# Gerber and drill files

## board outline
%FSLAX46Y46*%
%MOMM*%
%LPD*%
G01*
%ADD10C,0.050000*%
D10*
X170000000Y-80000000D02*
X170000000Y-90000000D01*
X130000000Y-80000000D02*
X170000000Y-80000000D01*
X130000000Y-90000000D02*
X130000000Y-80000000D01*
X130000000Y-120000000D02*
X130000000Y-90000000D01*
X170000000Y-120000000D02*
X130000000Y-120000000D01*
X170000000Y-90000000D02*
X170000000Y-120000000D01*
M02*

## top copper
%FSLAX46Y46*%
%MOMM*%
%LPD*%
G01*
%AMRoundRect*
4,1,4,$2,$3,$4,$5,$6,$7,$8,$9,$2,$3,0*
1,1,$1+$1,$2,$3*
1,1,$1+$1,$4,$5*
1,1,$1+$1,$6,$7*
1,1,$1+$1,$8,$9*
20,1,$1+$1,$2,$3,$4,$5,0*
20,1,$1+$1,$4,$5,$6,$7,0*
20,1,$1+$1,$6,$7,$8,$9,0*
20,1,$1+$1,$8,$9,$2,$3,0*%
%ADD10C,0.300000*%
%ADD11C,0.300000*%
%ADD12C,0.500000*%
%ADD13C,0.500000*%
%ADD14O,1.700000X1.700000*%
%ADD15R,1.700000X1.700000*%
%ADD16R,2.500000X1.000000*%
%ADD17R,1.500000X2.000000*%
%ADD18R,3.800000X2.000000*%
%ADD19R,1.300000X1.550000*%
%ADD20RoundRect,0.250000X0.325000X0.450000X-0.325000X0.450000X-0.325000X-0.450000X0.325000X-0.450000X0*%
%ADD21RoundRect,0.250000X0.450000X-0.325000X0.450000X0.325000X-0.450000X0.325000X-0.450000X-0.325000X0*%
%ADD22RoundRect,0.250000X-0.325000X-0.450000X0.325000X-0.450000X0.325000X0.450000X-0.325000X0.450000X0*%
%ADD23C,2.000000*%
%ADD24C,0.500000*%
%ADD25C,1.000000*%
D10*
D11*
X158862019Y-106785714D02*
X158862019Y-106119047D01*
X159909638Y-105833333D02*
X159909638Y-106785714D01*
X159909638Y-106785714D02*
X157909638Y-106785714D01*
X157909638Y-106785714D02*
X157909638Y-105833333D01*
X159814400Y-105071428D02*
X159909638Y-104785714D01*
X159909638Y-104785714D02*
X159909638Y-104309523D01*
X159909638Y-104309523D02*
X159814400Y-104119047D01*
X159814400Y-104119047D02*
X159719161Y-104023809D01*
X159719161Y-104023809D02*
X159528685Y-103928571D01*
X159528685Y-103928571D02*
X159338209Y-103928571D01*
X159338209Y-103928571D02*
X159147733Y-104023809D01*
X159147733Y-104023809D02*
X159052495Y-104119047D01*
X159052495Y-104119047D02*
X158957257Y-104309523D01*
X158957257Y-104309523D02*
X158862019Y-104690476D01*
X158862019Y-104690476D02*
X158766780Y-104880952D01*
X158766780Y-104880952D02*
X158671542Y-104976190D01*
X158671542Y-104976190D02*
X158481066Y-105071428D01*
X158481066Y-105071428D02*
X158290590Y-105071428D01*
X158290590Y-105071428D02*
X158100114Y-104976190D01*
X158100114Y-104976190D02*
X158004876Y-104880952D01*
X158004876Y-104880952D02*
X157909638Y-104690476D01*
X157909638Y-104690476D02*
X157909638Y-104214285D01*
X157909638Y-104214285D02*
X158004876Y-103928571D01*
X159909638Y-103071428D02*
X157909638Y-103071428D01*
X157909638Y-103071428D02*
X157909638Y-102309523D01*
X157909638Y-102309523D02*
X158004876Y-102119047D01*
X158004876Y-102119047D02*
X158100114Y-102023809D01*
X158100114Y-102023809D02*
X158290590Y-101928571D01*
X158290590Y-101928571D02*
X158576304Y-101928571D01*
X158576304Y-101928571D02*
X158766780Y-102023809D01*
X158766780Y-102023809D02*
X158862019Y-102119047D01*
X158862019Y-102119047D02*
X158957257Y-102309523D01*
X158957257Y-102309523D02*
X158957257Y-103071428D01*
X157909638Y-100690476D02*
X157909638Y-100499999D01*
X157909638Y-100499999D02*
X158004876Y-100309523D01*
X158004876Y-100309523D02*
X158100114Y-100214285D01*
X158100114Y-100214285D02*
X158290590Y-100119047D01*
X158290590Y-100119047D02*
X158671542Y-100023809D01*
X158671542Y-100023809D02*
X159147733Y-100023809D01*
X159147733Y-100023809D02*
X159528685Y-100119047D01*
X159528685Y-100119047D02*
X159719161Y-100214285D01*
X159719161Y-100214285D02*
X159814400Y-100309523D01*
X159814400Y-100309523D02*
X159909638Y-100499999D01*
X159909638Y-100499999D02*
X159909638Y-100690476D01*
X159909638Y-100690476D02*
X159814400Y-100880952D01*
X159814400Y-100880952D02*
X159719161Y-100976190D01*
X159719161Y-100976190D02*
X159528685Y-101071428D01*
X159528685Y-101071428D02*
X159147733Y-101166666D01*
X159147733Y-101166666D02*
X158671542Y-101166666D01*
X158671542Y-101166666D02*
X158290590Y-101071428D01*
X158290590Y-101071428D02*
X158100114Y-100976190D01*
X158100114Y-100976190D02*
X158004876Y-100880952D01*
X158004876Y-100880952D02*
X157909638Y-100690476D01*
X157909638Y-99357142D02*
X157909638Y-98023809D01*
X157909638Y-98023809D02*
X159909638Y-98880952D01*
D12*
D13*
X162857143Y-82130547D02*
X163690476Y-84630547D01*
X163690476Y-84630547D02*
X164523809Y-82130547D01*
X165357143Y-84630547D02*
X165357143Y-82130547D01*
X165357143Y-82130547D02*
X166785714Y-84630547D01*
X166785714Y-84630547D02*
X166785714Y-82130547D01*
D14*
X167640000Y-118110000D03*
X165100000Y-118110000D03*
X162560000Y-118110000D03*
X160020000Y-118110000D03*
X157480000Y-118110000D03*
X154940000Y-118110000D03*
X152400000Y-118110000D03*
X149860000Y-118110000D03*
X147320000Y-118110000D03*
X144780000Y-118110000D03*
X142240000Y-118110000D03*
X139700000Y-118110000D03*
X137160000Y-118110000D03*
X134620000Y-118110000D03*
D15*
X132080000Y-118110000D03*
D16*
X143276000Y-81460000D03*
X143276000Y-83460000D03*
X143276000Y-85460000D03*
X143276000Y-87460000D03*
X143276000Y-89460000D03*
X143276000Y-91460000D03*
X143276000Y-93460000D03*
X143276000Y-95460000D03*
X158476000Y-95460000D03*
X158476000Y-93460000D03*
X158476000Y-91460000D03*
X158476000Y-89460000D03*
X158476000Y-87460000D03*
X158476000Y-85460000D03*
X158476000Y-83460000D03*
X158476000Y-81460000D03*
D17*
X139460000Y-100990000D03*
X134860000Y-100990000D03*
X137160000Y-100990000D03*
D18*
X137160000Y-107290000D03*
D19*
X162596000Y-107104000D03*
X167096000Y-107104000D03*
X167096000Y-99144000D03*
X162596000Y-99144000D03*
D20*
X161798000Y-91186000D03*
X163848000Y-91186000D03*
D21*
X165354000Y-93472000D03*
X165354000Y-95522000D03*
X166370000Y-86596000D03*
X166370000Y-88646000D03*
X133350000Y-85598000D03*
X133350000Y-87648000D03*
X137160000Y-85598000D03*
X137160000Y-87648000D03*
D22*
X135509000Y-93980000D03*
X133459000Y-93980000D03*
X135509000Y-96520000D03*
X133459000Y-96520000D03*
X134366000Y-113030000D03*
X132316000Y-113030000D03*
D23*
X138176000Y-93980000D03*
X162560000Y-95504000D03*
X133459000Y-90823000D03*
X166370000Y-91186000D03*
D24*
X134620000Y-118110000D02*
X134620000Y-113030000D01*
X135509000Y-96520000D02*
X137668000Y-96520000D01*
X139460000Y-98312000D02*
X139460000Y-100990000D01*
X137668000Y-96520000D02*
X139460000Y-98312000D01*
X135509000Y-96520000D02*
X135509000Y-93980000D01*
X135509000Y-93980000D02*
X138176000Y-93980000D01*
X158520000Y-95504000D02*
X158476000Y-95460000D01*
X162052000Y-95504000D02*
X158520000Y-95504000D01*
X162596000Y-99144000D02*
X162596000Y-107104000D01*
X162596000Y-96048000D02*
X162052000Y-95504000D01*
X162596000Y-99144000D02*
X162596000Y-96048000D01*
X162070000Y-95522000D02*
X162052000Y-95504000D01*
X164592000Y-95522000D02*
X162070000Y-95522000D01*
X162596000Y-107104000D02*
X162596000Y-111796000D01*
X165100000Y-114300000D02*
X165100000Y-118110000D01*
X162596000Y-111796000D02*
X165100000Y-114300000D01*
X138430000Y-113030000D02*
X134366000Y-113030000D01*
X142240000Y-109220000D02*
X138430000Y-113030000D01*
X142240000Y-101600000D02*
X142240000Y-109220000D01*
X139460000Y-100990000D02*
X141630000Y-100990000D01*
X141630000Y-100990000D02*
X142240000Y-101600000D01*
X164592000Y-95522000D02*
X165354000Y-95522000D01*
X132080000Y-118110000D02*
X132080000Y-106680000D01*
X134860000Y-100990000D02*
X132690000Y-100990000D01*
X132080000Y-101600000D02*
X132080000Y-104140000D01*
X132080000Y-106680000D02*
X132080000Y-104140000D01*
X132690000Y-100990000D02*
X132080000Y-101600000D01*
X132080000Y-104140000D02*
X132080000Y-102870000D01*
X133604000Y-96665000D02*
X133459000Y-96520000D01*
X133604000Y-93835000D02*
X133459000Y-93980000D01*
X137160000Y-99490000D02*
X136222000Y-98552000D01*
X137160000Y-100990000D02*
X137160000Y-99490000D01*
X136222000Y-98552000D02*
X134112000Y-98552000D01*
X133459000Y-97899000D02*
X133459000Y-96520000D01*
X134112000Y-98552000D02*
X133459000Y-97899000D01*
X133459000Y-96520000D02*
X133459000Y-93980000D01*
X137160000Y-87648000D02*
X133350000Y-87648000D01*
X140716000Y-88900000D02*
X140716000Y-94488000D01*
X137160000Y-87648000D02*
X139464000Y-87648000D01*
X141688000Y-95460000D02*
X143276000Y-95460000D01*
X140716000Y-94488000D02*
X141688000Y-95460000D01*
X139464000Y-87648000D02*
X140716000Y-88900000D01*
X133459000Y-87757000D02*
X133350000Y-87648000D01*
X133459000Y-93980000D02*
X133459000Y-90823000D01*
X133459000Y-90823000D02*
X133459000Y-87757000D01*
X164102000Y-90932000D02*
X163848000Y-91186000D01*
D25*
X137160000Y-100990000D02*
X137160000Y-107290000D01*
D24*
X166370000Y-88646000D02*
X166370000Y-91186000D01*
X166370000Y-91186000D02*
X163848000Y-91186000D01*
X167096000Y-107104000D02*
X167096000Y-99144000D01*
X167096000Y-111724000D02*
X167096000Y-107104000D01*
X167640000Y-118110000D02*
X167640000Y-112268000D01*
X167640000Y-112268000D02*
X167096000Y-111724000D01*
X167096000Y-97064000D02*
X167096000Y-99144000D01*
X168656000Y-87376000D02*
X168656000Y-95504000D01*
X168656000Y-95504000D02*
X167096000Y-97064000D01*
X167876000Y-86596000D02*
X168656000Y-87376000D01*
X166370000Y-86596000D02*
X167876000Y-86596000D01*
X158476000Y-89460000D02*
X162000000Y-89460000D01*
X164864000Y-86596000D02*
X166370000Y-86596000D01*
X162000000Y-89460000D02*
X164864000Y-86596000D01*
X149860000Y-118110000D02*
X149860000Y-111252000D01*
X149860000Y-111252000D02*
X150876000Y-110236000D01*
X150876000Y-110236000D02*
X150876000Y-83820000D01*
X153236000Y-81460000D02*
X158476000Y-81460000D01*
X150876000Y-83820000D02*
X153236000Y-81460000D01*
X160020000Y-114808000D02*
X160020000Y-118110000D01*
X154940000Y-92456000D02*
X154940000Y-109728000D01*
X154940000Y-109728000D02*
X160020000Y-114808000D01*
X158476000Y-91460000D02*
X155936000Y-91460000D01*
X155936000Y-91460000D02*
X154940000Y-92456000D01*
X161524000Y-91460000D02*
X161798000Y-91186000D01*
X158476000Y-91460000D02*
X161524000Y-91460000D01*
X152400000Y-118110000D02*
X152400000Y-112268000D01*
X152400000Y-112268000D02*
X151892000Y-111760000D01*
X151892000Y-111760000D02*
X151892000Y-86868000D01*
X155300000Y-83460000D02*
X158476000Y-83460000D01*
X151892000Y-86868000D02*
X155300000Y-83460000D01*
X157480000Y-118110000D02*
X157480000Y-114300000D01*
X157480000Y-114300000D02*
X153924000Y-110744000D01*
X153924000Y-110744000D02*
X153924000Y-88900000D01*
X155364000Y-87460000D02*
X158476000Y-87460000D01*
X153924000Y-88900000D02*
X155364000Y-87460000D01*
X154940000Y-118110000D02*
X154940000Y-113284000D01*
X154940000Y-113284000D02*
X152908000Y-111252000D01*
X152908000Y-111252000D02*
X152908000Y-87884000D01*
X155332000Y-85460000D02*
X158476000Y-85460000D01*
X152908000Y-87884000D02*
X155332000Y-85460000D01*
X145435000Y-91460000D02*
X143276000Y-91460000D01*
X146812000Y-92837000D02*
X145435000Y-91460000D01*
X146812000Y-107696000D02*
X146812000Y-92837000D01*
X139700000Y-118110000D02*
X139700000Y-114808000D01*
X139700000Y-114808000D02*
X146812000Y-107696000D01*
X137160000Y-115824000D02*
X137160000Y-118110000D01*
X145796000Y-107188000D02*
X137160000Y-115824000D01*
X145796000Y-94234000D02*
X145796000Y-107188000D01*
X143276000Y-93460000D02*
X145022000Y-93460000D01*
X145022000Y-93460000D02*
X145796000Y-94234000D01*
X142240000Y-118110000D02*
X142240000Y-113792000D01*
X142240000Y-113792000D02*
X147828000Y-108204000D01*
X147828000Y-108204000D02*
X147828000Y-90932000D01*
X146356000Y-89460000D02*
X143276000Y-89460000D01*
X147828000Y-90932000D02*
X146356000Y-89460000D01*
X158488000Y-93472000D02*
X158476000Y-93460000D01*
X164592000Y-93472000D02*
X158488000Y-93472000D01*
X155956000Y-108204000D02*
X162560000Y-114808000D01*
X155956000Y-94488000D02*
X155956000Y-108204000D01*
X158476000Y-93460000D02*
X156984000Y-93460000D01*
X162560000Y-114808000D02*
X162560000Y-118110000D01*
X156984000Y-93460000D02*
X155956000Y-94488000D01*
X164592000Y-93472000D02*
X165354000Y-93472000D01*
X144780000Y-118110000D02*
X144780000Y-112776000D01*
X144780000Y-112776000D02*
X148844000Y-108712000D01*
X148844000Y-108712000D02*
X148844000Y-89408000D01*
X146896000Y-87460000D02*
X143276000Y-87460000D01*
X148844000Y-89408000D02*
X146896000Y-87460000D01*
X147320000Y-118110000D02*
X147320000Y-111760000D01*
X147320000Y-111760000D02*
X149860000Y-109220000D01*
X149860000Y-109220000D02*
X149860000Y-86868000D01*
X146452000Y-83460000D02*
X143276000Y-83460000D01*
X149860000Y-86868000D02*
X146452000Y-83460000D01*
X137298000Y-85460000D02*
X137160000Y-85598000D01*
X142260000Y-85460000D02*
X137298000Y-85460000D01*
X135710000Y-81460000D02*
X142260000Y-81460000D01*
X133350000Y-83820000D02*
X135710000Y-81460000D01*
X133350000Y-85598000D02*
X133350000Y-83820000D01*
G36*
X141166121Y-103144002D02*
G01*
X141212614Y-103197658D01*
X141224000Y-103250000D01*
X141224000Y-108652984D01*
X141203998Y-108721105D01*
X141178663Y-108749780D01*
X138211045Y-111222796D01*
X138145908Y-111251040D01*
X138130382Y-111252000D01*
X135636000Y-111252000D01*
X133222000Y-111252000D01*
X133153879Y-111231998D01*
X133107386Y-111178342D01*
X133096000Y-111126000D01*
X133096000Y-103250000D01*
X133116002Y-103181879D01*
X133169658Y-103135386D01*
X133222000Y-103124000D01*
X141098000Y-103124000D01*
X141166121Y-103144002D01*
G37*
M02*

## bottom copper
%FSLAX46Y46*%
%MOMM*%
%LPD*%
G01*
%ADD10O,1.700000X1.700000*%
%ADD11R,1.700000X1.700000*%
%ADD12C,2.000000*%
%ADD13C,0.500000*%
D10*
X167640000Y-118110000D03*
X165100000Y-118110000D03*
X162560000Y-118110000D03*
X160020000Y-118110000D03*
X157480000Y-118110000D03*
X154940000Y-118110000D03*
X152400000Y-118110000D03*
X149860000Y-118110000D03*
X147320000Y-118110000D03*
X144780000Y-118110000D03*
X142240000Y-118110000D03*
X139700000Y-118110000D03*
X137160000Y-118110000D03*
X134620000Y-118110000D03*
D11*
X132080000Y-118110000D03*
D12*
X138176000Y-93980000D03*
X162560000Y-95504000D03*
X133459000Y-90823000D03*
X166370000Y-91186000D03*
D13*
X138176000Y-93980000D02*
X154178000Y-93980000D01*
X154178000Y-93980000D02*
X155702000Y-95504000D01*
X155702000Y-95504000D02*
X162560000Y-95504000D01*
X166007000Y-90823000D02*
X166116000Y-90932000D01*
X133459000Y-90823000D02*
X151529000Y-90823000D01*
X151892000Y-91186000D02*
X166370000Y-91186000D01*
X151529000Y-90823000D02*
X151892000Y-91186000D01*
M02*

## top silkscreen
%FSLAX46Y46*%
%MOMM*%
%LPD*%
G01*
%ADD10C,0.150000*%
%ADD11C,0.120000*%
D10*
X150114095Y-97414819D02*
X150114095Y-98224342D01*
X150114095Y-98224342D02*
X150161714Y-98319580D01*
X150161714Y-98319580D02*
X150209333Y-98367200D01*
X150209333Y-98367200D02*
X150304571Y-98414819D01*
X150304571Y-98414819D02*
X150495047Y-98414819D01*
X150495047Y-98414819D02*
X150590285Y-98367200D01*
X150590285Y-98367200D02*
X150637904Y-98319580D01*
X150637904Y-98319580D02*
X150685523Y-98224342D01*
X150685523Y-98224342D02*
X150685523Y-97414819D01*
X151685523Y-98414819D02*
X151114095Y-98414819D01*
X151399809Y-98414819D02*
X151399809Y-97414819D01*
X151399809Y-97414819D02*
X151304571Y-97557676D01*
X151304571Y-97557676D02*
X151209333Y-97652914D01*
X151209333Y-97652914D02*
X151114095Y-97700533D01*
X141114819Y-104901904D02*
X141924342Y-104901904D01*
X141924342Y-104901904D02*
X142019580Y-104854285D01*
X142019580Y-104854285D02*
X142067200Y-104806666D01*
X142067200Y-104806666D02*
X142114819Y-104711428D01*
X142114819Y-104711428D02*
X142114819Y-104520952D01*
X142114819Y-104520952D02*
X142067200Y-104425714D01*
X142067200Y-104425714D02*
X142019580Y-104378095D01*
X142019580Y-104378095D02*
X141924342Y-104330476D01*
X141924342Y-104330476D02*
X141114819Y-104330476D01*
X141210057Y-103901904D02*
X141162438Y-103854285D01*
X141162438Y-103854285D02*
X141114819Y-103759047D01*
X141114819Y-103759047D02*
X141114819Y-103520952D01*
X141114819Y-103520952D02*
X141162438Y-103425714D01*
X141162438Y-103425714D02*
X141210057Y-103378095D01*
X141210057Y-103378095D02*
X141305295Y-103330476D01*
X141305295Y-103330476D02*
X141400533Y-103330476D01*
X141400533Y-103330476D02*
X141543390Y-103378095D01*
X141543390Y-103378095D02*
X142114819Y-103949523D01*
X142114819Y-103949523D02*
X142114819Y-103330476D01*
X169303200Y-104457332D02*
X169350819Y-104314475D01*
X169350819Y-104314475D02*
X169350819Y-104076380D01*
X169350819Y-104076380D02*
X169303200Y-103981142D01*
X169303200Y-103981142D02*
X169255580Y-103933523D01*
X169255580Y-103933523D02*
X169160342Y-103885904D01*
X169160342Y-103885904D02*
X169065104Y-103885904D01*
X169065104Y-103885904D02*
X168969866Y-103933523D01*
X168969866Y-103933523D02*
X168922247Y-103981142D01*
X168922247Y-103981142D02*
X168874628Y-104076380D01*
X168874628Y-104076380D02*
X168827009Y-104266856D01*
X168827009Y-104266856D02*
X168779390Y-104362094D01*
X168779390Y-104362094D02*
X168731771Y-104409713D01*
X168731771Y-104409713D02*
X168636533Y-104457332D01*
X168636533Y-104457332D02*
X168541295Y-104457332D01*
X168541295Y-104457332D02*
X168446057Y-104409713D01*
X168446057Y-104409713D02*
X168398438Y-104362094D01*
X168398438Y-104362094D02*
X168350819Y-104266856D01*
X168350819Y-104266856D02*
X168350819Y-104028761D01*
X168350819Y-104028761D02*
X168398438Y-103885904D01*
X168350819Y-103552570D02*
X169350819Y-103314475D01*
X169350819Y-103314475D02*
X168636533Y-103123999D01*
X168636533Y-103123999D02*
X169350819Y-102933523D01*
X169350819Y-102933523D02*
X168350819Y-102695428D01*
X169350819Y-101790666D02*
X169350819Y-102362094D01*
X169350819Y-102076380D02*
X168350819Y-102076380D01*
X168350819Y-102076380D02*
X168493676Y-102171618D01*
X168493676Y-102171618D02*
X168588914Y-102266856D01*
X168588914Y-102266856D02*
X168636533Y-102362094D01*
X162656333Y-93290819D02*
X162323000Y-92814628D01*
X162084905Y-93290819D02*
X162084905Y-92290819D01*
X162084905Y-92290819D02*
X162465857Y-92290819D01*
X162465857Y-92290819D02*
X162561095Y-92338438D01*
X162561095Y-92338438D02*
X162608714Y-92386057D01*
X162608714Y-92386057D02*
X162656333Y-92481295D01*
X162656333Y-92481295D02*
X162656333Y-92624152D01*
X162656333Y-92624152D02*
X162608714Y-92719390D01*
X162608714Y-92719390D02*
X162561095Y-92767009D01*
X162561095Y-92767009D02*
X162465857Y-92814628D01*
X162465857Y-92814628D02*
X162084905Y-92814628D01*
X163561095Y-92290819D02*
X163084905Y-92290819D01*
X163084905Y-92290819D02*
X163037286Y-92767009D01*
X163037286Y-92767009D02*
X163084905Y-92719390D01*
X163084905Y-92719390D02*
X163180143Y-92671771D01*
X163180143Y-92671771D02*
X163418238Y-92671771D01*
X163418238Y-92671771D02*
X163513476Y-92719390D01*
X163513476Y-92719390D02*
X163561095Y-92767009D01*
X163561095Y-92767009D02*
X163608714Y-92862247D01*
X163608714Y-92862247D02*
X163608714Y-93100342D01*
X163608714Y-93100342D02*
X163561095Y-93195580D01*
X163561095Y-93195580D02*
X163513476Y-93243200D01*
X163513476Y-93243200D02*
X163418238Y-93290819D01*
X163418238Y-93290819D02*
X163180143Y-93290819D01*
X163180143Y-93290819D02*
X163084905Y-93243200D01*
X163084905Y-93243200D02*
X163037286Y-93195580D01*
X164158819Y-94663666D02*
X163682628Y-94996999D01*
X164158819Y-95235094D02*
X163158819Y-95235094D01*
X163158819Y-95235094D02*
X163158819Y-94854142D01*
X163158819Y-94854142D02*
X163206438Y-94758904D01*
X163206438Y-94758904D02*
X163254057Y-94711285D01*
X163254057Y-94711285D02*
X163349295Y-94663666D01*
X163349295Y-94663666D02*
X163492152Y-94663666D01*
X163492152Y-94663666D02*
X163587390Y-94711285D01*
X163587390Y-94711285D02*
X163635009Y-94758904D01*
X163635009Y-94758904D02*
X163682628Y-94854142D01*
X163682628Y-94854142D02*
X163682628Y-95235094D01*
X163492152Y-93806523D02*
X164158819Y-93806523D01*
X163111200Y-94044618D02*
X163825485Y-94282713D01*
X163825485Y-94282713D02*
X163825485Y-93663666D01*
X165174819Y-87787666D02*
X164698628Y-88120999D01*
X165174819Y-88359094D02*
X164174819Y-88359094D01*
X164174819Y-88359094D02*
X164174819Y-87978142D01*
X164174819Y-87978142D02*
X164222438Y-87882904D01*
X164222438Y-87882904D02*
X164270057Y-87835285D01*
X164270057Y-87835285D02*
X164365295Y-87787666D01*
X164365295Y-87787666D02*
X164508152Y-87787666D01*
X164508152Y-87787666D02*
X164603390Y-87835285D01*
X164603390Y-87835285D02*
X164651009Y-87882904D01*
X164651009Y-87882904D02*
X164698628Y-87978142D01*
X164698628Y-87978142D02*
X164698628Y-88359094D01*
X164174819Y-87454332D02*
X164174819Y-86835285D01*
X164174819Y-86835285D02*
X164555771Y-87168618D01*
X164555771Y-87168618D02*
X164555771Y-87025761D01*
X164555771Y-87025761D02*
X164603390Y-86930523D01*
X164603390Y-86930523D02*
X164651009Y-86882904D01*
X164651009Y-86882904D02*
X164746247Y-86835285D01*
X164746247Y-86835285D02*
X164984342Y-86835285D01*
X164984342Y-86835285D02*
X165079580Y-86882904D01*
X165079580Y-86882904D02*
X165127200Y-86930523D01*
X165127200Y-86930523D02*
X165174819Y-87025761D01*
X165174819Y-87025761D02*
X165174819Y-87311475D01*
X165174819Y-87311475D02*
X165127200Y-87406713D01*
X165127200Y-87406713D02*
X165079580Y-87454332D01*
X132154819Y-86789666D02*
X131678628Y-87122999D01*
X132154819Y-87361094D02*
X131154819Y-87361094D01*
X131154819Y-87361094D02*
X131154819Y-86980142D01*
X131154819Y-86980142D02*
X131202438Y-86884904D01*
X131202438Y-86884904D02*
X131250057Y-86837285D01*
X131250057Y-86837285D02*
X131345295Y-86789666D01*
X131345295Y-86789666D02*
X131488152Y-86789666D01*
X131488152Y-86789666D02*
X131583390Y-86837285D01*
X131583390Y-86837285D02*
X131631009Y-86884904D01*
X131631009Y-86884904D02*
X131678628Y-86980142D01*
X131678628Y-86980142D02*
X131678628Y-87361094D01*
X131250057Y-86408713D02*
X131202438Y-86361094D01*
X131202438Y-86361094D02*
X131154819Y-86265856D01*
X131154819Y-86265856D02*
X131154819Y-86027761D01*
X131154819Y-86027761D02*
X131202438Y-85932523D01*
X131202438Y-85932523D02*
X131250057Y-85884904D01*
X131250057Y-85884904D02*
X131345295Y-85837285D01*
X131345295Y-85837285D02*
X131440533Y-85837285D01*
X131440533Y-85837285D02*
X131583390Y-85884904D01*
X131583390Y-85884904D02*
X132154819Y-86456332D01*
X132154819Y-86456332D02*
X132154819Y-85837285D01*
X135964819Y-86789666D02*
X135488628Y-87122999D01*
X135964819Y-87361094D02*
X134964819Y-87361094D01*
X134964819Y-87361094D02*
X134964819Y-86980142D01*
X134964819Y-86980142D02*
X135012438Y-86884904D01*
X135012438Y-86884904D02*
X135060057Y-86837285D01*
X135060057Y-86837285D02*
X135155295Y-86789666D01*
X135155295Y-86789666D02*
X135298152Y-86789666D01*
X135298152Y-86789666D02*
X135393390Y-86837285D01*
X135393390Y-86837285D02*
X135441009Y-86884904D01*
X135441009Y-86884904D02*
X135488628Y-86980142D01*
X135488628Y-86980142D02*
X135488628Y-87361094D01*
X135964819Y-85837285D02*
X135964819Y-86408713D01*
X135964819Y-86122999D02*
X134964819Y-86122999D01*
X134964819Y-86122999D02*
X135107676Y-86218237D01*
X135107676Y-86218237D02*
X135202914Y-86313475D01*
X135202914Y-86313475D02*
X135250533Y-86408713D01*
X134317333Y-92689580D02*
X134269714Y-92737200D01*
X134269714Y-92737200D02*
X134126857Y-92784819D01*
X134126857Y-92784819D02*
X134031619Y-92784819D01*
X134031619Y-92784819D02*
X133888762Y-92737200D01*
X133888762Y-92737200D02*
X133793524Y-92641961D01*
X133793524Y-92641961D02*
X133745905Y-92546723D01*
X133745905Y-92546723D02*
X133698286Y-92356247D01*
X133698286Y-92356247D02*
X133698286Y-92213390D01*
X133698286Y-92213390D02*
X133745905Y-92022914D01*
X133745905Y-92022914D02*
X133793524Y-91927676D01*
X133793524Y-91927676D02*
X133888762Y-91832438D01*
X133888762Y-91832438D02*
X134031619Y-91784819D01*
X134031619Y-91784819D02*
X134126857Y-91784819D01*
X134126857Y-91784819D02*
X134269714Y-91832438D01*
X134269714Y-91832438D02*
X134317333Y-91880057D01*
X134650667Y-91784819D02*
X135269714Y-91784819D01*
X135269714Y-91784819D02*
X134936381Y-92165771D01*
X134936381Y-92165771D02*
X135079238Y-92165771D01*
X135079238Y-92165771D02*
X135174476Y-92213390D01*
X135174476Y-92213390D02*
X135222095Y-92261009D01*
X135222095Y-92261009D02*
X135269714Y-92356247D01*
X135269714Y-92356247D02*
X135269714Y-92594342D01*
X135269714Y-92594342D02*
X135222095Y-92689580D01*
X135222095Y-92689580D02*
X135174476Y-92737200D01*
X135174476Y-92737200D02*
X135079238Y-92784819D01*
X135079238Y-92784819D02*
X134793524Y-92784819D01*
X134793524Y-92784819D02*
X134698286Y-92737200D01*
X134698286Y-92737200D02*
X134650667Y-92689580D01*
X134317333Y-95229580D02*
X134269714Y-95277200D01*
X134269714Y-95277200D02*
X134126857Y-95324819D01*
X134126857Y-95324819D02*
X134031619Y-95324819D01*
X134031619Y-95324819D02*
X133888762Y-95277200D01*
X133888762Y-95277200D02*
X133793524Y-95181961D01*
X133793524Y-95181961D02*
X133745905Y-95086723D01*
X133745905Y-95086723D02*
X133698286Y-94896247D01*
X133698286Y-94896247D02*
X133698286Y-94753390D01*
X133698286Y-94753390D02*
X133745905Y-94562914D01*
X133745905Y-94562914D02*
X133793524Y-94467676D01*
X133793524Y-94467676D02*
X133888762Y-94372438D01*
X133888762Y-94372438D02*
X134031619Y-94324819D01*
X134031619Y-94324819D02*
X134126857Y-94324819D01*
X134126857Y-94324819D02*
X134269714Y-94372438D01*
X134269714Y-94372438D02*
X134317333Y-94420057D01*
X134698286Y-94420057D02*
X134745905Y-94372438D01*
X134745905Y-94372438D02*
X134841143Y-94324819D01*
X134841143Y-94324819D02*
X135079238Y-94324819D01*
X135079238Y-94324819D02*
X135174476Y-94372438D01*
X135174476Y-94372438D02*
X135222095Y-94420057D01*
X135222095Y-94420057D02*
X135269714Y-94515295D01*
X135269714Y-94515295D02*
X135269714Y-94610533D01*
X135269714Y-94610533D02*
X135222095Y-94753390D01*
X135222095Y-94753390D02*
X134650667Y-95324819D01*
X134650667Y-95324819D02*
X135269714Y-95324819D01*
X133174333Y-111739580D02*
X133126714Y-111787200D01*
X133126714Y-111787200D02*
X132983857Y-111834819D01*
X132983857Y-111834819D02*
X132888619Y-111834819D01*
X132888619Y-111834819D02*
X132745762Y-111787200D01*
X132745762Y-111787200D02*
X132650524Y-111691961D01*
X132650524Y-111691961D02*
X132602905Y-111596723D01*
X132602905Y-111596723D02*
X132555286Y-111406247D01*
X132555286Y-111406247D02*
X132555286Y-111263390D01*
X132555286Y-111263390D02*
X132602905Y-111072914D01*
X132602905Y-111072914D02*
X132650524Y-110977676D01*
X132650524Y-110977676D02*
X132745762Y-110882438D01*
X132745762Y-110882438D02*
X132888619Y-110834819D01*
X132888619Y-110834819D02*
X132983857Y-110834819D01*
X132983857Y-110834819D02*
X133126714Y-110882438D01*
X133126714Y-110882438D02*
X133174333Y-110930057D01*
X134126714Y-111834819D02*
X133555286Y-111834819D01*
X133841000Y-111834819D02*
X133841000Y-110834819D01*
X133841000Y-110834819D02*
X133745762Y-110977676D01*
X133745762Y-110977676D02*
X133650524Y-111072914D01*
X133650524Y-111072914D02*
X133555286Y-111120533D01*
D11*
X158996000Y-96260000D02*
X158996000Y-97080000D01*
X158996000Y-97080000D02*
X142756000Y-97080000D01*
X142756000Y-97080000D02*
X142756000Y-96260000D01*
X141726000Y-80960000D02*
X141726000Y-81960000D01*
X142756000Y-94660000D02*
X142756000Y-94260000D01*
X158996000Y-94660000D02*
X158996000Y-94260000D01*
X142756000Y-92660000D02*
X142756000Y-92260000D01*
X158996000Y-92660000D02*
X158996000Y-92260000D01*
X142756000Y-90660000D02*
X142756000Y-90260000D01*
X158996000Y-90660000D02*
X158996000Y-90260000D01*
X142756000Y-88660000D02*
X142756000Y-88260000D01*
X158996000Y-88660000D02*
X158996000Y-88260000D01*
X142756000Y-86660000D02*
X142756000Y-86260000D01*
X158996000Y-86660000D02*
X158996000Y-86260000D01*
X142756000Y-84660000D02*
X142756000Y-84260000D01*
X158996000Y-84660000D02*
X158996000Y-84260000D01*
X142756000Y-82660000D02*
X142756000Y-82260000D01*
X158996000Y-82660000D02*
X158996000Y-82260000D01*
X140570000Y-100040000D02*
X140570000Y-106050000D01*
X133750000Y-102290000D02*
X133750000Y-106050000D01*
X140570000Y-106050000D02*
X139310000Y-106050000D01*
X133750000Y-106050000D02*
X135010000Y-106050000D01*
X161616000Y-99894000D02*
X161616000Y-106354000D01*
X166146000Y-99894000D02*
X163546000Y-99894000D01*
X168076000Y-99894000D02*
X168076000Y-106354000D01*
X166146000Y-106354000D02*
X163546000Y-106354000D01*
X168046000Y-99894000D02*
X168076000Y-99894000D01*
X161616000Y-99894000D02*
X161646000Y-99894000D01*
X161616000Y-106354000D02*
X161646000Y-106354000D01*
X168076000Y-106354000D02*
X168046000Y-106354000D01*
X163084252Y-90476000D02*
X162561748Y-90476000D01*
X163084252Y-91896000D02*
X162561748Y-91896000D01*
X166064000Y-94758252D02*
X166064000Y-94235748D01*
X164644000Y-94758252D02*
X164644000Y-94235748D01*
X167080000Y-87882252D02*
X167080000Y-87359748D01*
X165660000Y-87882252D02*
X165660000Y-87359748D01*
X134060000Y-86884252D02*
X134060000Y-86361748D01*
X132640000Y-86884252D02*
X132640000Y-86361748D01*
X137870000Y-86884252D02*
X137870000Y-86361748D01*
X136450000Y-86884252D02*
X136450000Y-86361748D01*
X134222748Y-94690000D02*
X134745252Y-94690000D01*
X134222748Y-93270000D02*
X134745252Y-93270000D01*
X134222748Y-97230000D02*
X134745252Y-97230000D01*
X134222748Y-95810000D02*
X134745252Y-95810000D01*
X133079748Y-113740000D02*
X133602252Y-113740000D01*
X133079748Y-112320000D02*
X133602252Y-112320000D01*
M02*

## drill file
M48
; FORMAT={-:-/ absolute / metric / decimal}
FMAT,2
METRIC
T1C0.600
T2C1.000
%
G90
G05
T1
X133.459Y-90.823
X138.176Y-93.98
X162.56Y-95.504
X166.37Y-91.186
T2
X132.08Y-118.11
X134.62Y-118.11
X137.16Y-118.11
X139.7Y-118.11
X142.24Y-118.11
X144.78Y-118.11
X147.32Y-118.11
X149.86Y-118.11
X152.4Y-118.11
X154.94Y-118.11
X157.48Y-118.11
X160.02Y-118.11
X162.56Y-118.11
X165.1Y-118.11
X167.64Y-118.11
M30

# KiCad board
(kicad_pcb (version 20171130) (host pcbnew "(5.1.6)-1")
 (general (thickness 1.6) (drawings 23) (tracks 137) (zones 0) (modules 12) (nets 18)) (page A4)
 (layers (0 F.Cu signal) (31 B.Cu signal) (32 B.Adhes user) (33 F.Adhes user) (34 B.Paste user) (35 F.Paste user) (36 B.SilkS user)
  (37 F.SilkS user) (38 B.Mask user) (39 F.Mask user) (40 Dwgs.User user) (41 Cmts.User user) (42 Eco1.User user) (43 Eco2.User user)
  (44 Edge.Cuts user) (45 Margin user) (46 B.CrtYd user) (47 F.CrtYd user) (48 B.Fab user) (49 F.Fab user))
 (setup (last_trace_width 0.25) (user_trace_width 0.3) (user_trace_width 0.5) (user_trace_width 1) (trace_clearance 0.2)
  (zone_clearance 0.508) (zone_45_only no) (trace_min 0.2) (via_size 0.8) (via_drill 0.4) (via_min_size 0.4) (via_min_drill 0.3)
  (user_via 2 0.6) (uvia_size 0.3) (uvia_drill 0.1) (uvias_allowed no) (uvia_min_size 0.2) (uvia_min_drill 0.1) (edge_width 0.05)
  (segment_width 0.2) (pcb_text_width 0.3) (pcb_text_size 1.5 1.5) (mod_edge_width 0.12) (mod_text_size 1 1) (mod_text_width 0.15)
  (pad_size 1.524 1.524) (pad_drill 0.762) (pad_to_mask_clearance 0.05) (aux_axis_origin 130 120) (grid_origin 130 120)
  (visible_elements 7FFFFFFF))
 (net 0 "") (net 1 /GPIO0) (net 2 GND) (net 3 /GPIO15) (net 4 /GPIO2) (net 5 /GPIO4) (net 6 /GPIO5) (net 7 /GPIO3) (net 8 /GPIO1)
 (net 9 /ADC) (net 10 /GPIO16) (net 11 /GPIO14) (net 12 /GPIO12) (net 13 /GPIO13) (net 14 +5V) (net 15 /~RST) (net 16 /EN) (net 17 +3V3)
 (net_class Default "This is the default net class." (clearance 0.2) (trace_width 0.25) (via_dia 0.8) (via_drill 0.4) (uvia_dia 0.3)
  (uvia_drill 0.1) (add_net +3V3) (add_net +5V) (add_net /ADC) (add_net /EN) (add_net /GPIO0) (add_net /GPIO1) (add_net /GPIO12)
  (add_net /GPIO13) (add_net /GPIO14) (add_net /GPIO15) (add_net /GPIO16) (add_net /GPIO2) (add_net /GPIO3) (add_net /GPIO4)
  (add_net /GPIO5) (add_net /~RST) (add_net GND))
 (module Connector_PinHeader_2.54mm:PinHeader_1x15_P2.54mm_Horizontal (layer B.Cu) (at 132.08 118.11 270)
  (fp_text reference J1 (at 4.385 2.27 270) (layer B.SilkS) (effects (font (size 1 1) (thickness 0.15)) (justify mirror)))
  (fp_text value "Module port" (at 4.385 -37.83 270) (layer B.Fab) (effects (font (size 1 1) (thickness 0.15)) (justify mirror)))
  (pad 15 thru_hole oval (at 0 -35.56 270) (size 1.7 1.7) (drill 1) (layers *.Cu *.Mask) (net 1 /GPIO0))
  (pad 14 thru_hole oval (at 0 -33.02 270) (size 1.7 1.7) (drill 1) (layers *.Cu *.Mask) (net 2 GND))
  (pad 13 thru_hole oval (at 0 -30.48 270) (size 1.7 1.7) (drill 1) (layers *.Cu *.Mask) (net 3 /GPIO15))
  (pad 12 thru_hole oval (at 0 -27.94 270) (size 1.7 1.7) (drill 1) (layers *.Cu *.Mask) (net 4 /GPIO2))
  (pad 11 thru_hole oval (at 0 -25.4 270) (size 1.7 1.7) (drill 1) (layers *.Cu *.Mask) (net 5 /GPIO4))
  (pad 10 thru_hole oval (at 0 -22.86 270) (size 1.7 1.7) (drill 1) (layers *.Cu *.Mask) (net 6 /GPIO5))
  (pad 9 thru_hole oval (at 0 -20.32 270) (size 1.7 1.7) (drill 1) (layers *.Cu *.Mask) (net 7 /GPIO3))
  (pad 8 thru_hole oval (at 0 -17.78 270) (size 1.7 1.7) (drill 1) (layers *.Cu *.Mask) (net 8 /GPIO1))
  (pad 7 thru_hole oval (at 0 -15.24 270) (size 1.7 1.7) (drill 1) (layers *.Cu *.Mask) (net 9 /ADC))
  (pad 6 thru_hole oval (at 0 -12.7 270) (size 1.7 1.7) (drill 1) (layers *.Cu *.Mask) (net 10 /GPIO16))
  (pad 5 thru_hole oval (at 0 -10.16 270) (size 1.7 1.7) (drill 1) (layers *.Cu *.Mask) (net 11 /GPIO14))
  (pad 4 thru_hole oval (at 0 -7.62 270) (size 1.7 1.7) (drill 1) (layers *.Cu *.Mask) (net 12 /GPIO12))
  (pad 3 thru_hole oval (at 0 -5.08 270) (size 1.7 1.7) (drill 1) (layers *.Cu *.Mask) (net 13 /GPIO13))
  (pad 2 thru_hole oval (at 0 -2.54 270) (size 1.7 1.7) (drill 1) (layers *.Cu *.Mask) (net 2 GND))
  (pad 1 thru_hole rect (at 0 0 270) (size 1.7 1.7) (drill 1) (layers *.Cu *.Mask) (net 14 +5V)))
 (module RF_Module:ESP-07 (layer F.Cu) (at 150.876 86.36)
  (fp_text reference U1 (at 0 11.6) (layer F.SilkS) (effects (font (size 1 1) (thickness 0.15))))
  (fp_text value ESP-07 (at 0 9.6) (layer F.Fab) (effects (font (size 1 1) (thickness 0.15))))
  (fp_line (start 8.12 9.9) (end 8.12 10.72) (layer F.SilkS) (width 0.12))
  (fp_line (start 8.12 10.72) (end -8.12 10.72) (layer F.SilkS) (width 0.12))
  (fp_line (start -8.12 10.72) (end -8.12 9.9) (layer F.SilkS) (width 0.12))
  (fp_line (start -9.15 -5.4) (end -9.15 -4.4) (layer F.SilkS) (width 0.12))
  (fp_line (start -8.12 8.3) (end -8.12 7.9) (layer F.SilkS) (width 0.12))
  (fp_line (start 8.12 8.3) (end 8.12 7.9) (layer F.SilkS) (width 0.12))
  (fp_line (start -8.12 6.3) (end -8.12 5.9) (layer F.SilkS) (width 0.12))
  (fp_line (start 8.12 6.3) (end 8.12 5.9) (layer F.SilkS) (width 0.12))
  (fp_line (start -8.12 4.3) (end -8.12 3.9) (layer F.SilkS) (width 0.12))
  (fp_line (start 8.12 4.3) (end 8.12 3.9) (layer F.SilkS) (width 0.12))
  (fp_line (start -8.12 2.3) (end -8.12 1.9) (layer F.SilkS) (width 0.12))
  (fp_line (start 8.12 2.3) (end 8.12 1.9) (layer F.SilkS) (width 0.12))
  (fp_line (start -8.12 0.3) (end -8.12 -0.1) (layer F.SilkS) (width 0.12))
  (fp_line (start 8.12 0.3) (end 8.12 -0.1) (layer F.SilkS) (width 0.12))
  (fp_line (start -8.12 -1.7) (end -8.12 -2.1) (layer F.SilkS) (width 0.12))
  (fp_line (start 8.12 -1.7) (end 8.12 -2.1) (layer F.SilkS) (width 0.12))
  (fp_line (start -8.12 -3.7) (end -8.12 -4.1) (layer F.SilkS) (width 0.12))
  (fp_line (start 8.12 -3.7) (end 8.12 -4.1) (layer F.SilkS) (width 0.12))
  (pad 1 smd rect (at -7.6 -4.9) (size 2.5 1) (layers F.Cu F.Paste F.Mask) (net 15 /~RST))
  (pad 2 smd rect (at -7.6 -2.9) (size 2.5 1) (layers F.Cu F.Paste F.Mask) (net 9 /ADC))
  (pad 3 smd rect (at -7.6 -0.9) (size 2.5 1) (layers F.Cu F.Paste F.Mask) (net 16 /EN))
  (pad 4 smd rect (at -7.6 1.1) (size 2.5 1) (layers F.Cu F.Paste F.Mask) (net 10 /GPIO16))
  (pad 5 smd rect (at -7.6 3.1) (size 2.5 1) (layers F.Cu F.Paste F.Mask) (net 11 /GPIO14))
  (pad 6 smd rect (at -7.6 5.1) (size 2.5 1) (layers F.Cu F.Paste F.Mask) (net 12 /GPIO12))
  (pad 7 smd rect (at -7.6 7.1) (size 2.5 1) (layers F.Cu F.Paste F.Mask) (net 13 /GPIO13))
  (pad 8 smd rect (at -7.6 9.1) (size 2.5 1) (layers F.Cu F.Paste F.Mask) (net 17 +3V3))
  (pad 9 smd rect (at 7.6 9.1) (size 2.5 1) (layers F.Cu F.Paste F.Mask) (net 2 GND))
  (pad 10 smd rect (at 7.6 7.1) (size 2.5 1) (layers F.Cu F.Paste F.Mask) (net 3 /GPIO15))
  (pad 11 smd rect (at 7.6 5.1) (size 2.5 1) (layers F.Cu F.Paste F.Mask) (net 4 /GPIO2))
  (pad 12 smd rect (at 7.6 3.1) (size 2.5 1) (layers F.Cu F.Paste F.Mask) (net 1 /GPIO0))
  (pad 13 smd rect (at 7.6 1.1) (size 2.5 1) (layers F.Cu F.Paste F.Mask) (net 5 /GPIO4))
  (pad 14 smd rect (at 7.6 -0.9) (size 2.5 1) (layers F.Cu F.Paste F.Mask) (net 6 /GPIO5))
  (pad 15 smd rect (at 7.6 -2.9) (size 2.5 1) (layers F.Cu F.Paste F.Mask) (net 7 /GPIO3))
  (pad 16 smd rect (at 7.6 -4.9) (size 2.5 1) (layers F.Cu F.Paste F.Mask) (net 8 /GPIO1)))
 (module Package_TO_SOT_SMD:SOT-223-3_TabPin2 (layer F.Cu) (at 137.16 104.14 270)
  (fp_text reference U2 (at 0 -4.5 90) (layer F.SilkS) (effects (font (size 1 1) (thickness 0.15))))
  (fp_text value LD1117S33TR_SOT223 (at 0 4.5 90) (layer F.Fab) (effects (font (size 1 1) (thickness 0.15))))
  (fp_line (start -4.1 -3.41) (end 1.91 -3.41) (layer F.SilkS) (width 0.12))
  (fp_line (start -1.85 3.41) (end 1.91 3.41) (layer F.SilkS) (width 0.12))
  (fp_line (start 1.91 -3.41) (end 1.91 -2.15) (layer F.SilkS) (width 0.12))
  (fp_line (start 1.91 3.41) (end 1.91 2.15) (layer F.SilkS) (width 0.12))
  (pad 1 smd rect (at -3.15 -2.3 270) (size 2 1.5) (layers F.Cu F.Paste F.Mask) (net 2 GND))
  (pad 3 smd rect (at -3.15 2.3 270) (size 2 1.5) (layers F.Cu F.Paste F.Mask) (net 14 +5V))
  (pad 2 smd rect (at -3.15 0 270) (size 2 1.5) (layers F.Cu F.Paste F.Mask) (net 17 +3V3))
  (pad 2 smd rect (at 3.15 0 270) (size 2 3.8) (layers F.Cu F.Paste F.Mask) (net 17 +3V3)))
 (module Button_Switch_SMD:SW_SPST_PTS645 (layer F.Cu) (at 164.846 103.124 270)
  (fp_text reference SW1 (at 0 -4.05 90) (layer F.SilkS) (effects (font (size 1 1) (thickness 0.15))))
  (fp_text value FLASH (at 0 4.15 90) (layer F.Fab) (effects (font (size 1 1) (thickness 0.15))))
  (fp_line (start -3.23 3.23) (end 3.23 3.23) (layer F.SilkS) (width 0.12))
  (fp_line (start -3.23 -1.3) (end -3.23 1.3) (layer F.SilkS) (width 0.12))
  (fp_line (start -3.23 -3.23) (end 3.23 -3.23) (layer F.SilkS) (width 0.12))
  (fp_line (start 3.23 -1.3) (end 3.23 1.3) (layer F.SilkS) (width 0.12))
  (fp_line (start -3.23 -3.2) (end -3.23 -3.23) (layer F.SilkS) (width 0.12))
  (fp_line (start -3.23 3.23) (end -3.23 3.2) (layer F.SilkS) (width 0.12))
  (fp_line (start 3.23 3.23) (end 3.23 3.2) (layer F.SilkS) (width 0.12))
  (fp_line (start 3.23 -3.23) (end 3.23 -3.2) (layer F.SilkS) (width 0.12))
  (pad 2 smd rect (at 3.98 2.25 270) (size 1.55 1.3) (layers F.Cu F.Paste F.Mask) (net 2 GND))
  (pad 1 smd rect (at 3.98 -2.25 270) (size 1.55 1.3) (layers F.Cu F.Paste F.Mask) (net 1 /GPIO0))
  (pad 1 smd rect (at -3.98 -2.25 270) (size 1.55 1.3) (layers F.Cu F.Paste F.Mask) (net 1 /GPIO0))
  (pad 2 smd rect (at -3.98 2.25 270) (size 1.55 1.3) (layers F.Cu F.Paste F.Mask) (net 2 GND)))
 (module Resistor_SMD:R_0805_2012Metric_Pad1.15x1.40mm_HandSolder (layer F.Cu) (at 162.823 91.186 180)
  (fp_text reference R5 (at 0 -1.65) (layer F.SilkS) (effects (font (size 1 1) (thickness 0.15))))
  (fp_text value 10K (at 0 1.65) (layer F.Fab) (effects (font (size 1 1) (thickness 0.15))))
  (fp_line (start -0.261252 0.71) (end 0.261252 0.71) (layer F.SilkS) (width 0.12))
  (fp_line (start -0.261252 -0.71) (end 0.261252 -0.71) (layer F.SilkS) (width 0.12))
  (pad 2 smd roundrect (at 1.025 0 180) (size 1.15 1.4) (layers F.Cu F.Paste F.Mask) (roundrect_rratio 0.217391) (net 4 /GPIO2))
  (pad 1 smd roundrect (at -1.025 0 180) (size 1.15 1.4) (layers F.Cu F.Paste F.Mask) (roundrect_rratio 0.217391) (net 17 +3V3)))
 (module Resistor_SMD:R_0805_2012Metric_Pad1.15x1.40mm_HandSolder (layer F.Cu) (at 165.354 94.497 90)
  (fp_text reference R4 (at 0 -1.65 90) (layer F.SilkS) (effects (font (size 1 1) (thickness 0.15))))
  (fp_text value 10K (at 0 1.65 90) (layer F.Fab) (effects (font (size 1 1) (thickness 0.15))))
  (fp_line (start -0.261252 0.71) (end 0.261252 0.71) (layer F.SilkS) (width 0.12))
  (fp_line (start -0.261252 -0.71) (end 0.261252 -0.71) (layer F.SilkS) (width 0.12))
  (pad 2 smd roundrect (at 1.025 0 90) (size 1.15 1.4) (layers F.Cu F.Paste F.Mask) (roundrect_rratio 0.217391) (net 3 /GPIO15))
  (pad 1 smd roundrect (at -1.025 0 90) (size 1.15 1.4) (layers F.Cu F.Paste F.Mask) (roundrect_rratio 0.217391) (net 2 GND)))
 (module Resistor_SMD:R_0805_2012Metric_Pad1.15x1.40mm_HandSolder (layer F.Cu) (at 166.37 87.621 90)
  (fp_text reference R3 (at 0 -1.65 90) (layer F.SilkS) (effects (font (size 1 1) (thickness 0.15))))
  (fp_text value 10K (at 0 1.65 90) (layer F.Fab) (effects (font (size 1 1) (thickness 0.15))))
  (fp_line (start -0.261252 0.71) (end 0.261252 0.71) (layer F.SilkS) (width 0.12))
  (fp_line (start -0.261252 -0.71) (end 0.261252 -0.71) (layer F.SilkS) (width 0.12))
  (pad 2 smd roundrect (at 1.025 0 90) (size 1.15 1.4) (layers F.Cu F.Paste F.Mask) (roundrect_rratio 0.217391) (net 1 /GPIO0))
  (pad 1 smd roundrect (at -1.025 0 90) (size 1.15 1.4) (layers F.Cu F.Paste F.Mask) (roundrect_rratio 0.217391) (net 17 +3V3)))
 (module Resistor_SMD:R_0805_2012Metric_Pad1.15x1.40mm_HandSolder (layer F.Cu) (at 133.35 86.623 90)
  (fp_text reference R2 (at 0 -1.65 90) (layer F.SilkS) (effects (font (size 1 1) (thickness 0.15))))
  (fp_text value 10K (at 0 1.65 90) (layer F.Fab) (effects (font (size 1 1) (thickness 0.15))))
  (fp_line (start -0.261252 0.71) (end 0.261252 0.71) (layer F.SilkS) (width 0.12))
  (fp_line (start -0.261252 -0.71) (end 0.261252 -0.71) (layer F.SilkS) (width 0.12))
  (pad 2 smd roundrect (at 1.025 0 90) (size 1.15 1.4) (layers F.Cu F.Paste F.Mask) (roundrect_rratio 0.217391) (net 15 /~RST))
  (pad 1 smd roundrect (at -1.025 0 90) (size 1.15 1.4) (layers F.Cu F.Paste F.Mask) (roundrect_rratio 0.217391) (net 17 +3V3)))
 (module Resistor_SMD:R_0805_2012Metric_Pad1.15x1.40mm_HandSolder (layer F.Cu) (at 137.16 86.623 90)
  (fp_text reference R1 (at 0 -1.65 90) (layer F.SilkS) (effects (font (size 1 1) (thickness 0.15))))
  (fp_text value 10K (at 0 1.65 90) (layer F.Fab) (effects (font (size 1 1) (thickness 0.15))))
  (fp_line (start -0.261252 0.71) (end 0.261252 0.71) (layer F.SilkS) (width 0.12))
  (fp_line (start -0.261252 -0.71) (end 0.261252 -0.71) (layer F.SilkS) (width 0.12))
  (pad 2 smd roundrect (at 1.025 0 90) (size 1.15 1.4) (layers F.Cu F.Paste F.Mask) (roundrect_rratio 0.217391) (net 16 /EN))
  (pad 1 smd roundrect (at -1.025 0 90) (size 1.15 1.4) (layers F.Cu F.Paste F.Mask) (roundrect_rratio 0.217391) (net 17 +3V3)))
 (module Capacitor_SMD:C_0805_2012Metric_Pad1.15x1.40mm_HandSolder (layer F.Cu) (at 134.484 93.98)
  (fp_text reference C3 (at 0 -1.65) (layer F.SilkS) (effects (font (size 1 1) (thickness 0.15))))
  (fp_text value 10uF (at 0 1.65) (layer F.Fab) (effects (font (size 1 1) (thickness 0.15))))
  (fp_line (start -0.261252 0.71) (end 0.261252 0.71) (layer F.SilkS) (width 0.12))
  (fp_line (start -0.261252 -0.71) (end 0.261252 -0.71) (layer F.SilkS) (width 0.12))
  (pad 2 smd roundrect (at 1.025 0) (size 1.15 1.4) (layers F.Cu F.Paste F.Mask) (roundrect_rratio 0.217391) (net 2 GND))
  (pad 1 smd roundrect (at -1.025 0) (size 1.15 1.4) (layers F.Cu F.Paste F.Mask) (roundrect_rratio 0.217391) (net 17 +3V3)))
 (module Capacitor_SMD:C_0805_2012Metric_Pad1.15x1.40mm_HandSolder (layer F.Cu) (at 134.484 96.52)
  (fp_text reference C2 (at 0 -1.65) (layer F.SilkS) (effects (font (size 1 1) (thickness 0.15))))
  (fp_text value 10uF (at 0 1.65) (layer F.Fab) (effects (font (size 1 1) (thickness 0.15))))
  (fp_line (start -0.261252 0.71) (end 0.261252 0.71) (layer F.SilkS) (width 0.12))
  (fp_line (start -0.261252 -0.71) (end 0.261252 -0.71) (layer F.SilkS) (width 0.12))
  (pad 2 smd roundrect (at 1.025 0) (size 1.15 1.4) (layers F.Cu F.Paste F.Mask) (roundrect_rratio 0.217391) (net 2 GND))
  (pad 1 smd roundrect (at -1.025 0) (size 1.15 1.4) (layers F.Cu F.Paste F.Mask) (roundrect_rratio 0.217391) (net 17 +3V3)))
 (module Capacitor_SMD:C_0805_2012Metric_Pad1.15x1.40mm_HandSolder (layer F.Cu) (at 133.341 113.03)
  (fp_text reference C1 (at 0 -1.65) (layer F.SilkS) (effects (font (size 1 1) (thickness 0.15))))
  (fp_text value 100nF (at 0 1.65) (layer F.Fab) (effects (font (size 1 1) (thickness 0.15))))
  (fp_line (start -0.261252 0.71) (end 0.261252 0.71) (layer F.SilkS) (width 0.12))
  (fp_line (start -0.261252 -0.71) (end 0.261252 -0.71) (layer F.SilkS) (width 0.12))
  (pad 2 smd roundrect (at 1.025 0) (size 1.15 1.4) (layers F.Cu F.Paste F.Mask) (roundrect_rratio 0.217391) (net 2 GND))
  (pad 1 smd roundrect (at -1.025 0) (size 1.15 1.4) (layers F.Cu F.Paste F.Mask) (roundrect_rratio 0.217391) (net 14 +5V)))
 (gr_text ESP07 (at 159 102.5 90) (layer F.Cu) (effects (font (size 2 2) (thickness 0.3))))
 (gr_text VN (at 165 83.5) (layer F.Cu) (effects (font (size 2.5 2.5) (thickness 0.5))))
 (gr_line (start 170 80) (end 170 90) (layer Edge.Cuts) (width 0.05))
 (gr_line (start 130 80) (end 170 80) (layer Edge.Cuts) (width 0.05))
 (gr_line (start 130 90) (end 130 80) (layer Edge.Cuts) (width 0.05))
 (gr_line (start 130 120) (end 130 90) (layer Edge.Cuts) (width 0.05))
 (gr_line (start 170 120) (end 130 120) (layer Edge.Cuts) (width 0.05))
 (gr_line (start 170 90) (end 170 120) (layer Edge.Cuts) (width 0.05))
 (segment (start 134.62 118.11) (end 134.62 113.03) (width 0.5) (layer F.Cu) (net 2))
 (segment (start 135.509 96.52) (end 137.668 96.52) (width 0.5) (layer F.Cu) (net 2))
 (segment (start 139.46 98.312) (end 139.46 100.99) (width 0.5) (layer F.Cu) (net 2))
 (segment (start 137.668 96.52) (end 139.46 98.312) (width 0.5) (layer F.Cu) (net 2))
 (segment (start 135.509 96.52) (end 135.509 93.98) (width 0.5) (layer F.Cu) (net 2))
 (via (at 138.176 93.98) (size 2) (drill 0.6) (layers F.Cu B.Cu) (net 2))
 (segment (start 135.509 93.98) (end 138.176 93.98) (width 0.5) (layer F.Cu) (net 2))
 (segment (start 138.176 93.98) (end 154.178 93.98) (width 0.5) (layer B.Cu) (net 2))
 (via (at 162.56 95.504) (size 2) (drill 0.6) (layers F.Cu B.Cu) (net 2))
 (segment (start 154.178 93.98) (end 155.702 95.504) (width 0.5) (layer B.Cu) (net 2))
 (segment (start 158.52 95.504) (end 158.476 95.46) (width 0.5) (layer F.Cu) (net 2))
 (segment (start 162.052 95.504) (end 158.52 95.504) (width 0.5) (layer F.Cu) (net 2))
 (segment (start 162.596 99.144) (end 162.596 107.104) (width 0.5) (layer F.Cu) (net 2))
 (segment (start 162.596 96.048) (end 162.052 95.504) (width 0.5) (layer F.Cu) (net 2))
 (segment (start 162.596 99.144) (end 162.596 96.048) (width 0.5) (layer F.Cu) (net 2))
 (segment (start 162.07 95.522) (end 162.052 95.504) (width 0.5) (layer F.Cu) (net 2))
 (segment (start 164.592 95.522) (end 162.07 95.522) (width 0.5) (layer F.Cu) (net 2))
 (segment (start 162.596 107.104) (end 162.596 111.796) (width 0.5) (layer F.Cu) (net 2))
 (segment (start 165.1 114.3) (end 165.1 118.11) (width 0.5) (layer F.Cu) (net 2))
 (segment (start 162.596 111.796) (end 165.1 114.3) (width 0.5) (layer F.Cu) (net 2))
 (segment (start 138.43 113.03) (end 134.366 113.03) (width 0.5) (layer F.Cu) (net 2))
 (segment (start 142.24 109.22) (end 138.43 113.03) (width 0.5) (layer F.Cu) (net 2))
 (segment (start 142.24 101.6) (end 142.24 109.22) (width 0.5) (layer F.Cu) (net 2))
 (segment (start 139.46 100.99) (end 141.63 100.99) (width 0.5) (layer F.Cu) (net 2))
 (segment (start 141.63 100.99) (end 142.24 101.6) (width 0.5) (layer F.Cu) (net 2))
 (segment (start 164.592 95.522) (end 165.354 95.522) (width 0.5) (layer F.Cu) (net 2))
 (segment (start 155.702 95.504) (end 162.56 95.504) (width 0.5) (layer B.Cu) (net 2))
 (segment (start 132.08 118.11) (end 132.08 106.68) (width 0.5) (layer F.Cu) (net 14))
 (segment (start 134.86 100.99) (end 132.69 100.99) (width 0.5) (layer F.Cu) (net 14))
 (segment (start 132.08 101.6) (end 132.08 104.14) (width 0.5) (layer F.Cu) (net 14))
 (segment (start 132.08 106.68) (end 132.08 104.14) (width 0.5) (layer F.Cu) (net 14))
 (segment (start 132.69 100.99) (end 132.08 101.6) (width 0.5) (layer F.Cu) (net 14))
 (segment (start 132.08 104.14) (end 132.08 102.87) (width 0.5) (layer F.Cu) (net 14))
 (segment (start 133.604 96.665) (end 133.459 96.52) (width 0.5) (layer F.Cu) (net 17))
 (segment (start 133.604 93.835) (end 133.459 93.98) (width 0.5) (layer F.Cu) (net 17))
 (segment (start 137.16 99.49) (end 136.222 98.552) (width 0.5) (layer F.Cu) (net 17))
 (segment (start 137.16 100.99) (end 137.16 99.49) (width 0.5) (layer F.Cu) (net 17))
 (segment (start 136.222 98.552) (end 134.112 98.552) (width 0.5) (layer F.Cu) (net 17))
 (segment (start 133.459 97.899) (end 133.459 96.52) (width 0.5) (layer F.Cu) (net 17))
 (segment (start 134.112 98.552) (end 133.459 97.899) (width 0.5) (layer F.Cu) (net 17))
 (segment (start 133.459 96.52) (end 133.459 93.98) (width 0.5) (layer F.Cu) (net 17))
 (segment (start 137.16 87.648) (end 133.35 87.648) (width 0.5) (layer F.Cu) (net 17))
 (segment (start 140.716 88.9) (end 140.716 94.488) (width 0.5) (layer F.Cu) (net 17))
 (segment (start 137.16 87.648) (end 139.464 87.648) (width 0.5) (layer F.Cu) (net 17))
 (segment (start 141.688 95.46) (end 143.276 95.46) (width 0.5) (layer F.Cu) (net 17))
 (segment (start 140.716 94.488) (end 141.688 95.46) (width 0.5) (layer F.Cu) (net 17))
 (segment (start 139.464 87.648) (end 140.716 88.9) (width 0.5) (layer F.Cu) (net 17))
 (segment (start 133.459 87.757) (end 133.35 87.648) (width 0.5) (layer F.Cu) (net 17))
 (segment (start 133.459 93.98) (end 133.459 90.823) (width 0.5) (layer F.Cu) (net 17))
 (segment (start 133.459 90.823) (end 133.459 87.757) (width 0.5) (layer F.Cu) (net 17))
 (via (at 133.459 90.823) (size 2) (drill 0.6) (layers F.Cu B.Cu) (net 17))
 (via (at 166.37 91.186) (size 2) (drill 0.6) (layers F.Cu B.Cu) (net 17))
 (segment (start 166.007 90.823) (end 166.116 90.932) (width 0.5) (layer B.Cu) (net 17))
 (segment (start 164.102 90.932) (end 163.848 91.186) (width 0.5) (layer F.Cu) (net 17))
 (segment (start 137.16 100.99) (end 137.16 107.29) (width 1) (layer F.Cu) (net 17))
 (segment (start 166.37 88.646) (end 166.37 91.186) (width 0.5) (layer F.Cu) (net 17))
 (segment (start 166.37 91.186) (end 163.848 91.186) (width 0.5) (layer F.Cu) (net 17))
 (segment (start 133.459 90.823) (end 151.529 90.823) (width 0.5) (layer B.Cu) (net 17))
 (segment (start 151.892 91.186) (end 166.37 91.186) (width 0.5) (layer B.Cu) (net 17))
 (segment (start 151.529 90.823) (end 151.892 91.186) (width 0.5) (layer B.Cu) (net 17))
 (segment (start 167.096 107.104) (end 167.096 99.144) (width 0.5) (layer F.Cu) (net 1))
 (segment (start 167.096 111.724) (end 167.096 107.104) (width 0.5) (layer F.Cu) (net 1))
 (segment (start 167.64 118.11) (end 167.64 112.268) (width 0.5) (layer F.Cu) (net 1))
 (segment (start 167.64 112.268) (end 167.096 111.724) (width 0.5) (layer F.Cu) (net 1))
 (segment (start 167.096 97.064) (end 167.096 99.144) (width 0.5) (layer F.Cu) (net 1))
 (segment (start 168.656 87.376) (end 168.656 95.504) (width 0.5) (layer F.Cu) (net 1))
 (segment (start 168.656 95.504) (end 167.096 97.064) (width 0.5) (layer F.Cu) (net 1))
 (segment (start 167.876 86.596) (end 168.656 87.376) (width 0.5) (layer F.Cu) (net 1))
 (segment (start 166.37 86.596) (end 167.876 86.596) (width 0.5) (layer F.Cu) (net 1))
 (segment (start 158.476 89.46) (end 162 89.46) (width 0.5) (layer F.Cu) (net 1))
 (segment (start 164.864 86.596) (end 166.37 86.596) (width 0.5) (layer F.Cu) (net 1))
 (segment (start 162 89.46) (end 164.864 86.596) (width 0.5) (layer F.Cu) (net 1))
 (segment (start 149.86 118.11) (end 149.86 111.252) (width 0.5) (layer F.Cu) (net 8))
 (segment (start 149.86 111.252) (end 150.876 110.236) (width 0.5) (layer F.Cu) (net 8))
 (segment (start 150.876 110.236) (end 150.876 83.82) (width 0.5) (layer F.Cu) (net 8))
 (segment (start 153.236 81.46) (end 158.476 81.46) (width 0.5) (layer F.Cu) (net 8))
 (segment (start 150.876 83.82) (end 153.236 81.46) (width 0.5) (layer F.Cu) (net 8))
 (segment (start 160.02 114.808) (end 160.02 118.11) (width 0.5) (layer F.Cu) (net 4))
 (segment (start 154.94 92.456) (end 154.94 109.728) (width 0.5) (layer F.Cu) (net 4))
 (segment (start 154.94 109.728) (end 160.02 114.808) (width 0.5) (layer F.Cu) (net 4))
 (segment (start 158.476 91.46) (end 155.936 91.46) (width 0.5) (layer F.Cu) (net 4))
 (segment (start 155.936 91.46) (end 154.94 92.456) (width 0.5) (layer F.Cu) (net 4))
 (segment (start 161.524 91.46) (end 161.798 91.186) (width 0.5) (layer F.Cu) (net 4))
 (segment (start 158.476 91.46) (end 161.524 91.46) (width 0.5) (layer F.Cu) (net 4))
 (segment (start 152.4 118.11) (end 152.4 112.268) (width 0.5) (layer F.Cu) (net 7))
 (segment (start 152.4 112.268) (end 151.892 111.76) (width 0.5) (layer F.Cu) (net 7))
 (segment (start 151.892 111.76) (end 151.892 86.868) (width 0.5) (layer F.Cu) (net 7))
 (segment (start 155.3 83.46) (end 158.476 83.46) (width 0.5) (layer F.Cu) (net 7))
 (segment (start 151.892 86.868) (end 155.3 83.46) (width 0.5) (layer F.Cu) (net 7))
 (segment (start 157.48 118.11) (end 157.48 114.3) (width 0.5) (layer F.Cu) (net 5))
 (segment (start 157.48 114.3) (end 153.924 110.744) (width 0.5) (layer F.Cu) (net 5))
 (segment (start 153.924 110.744) (end 153.924 88.9) (width 0.5) (layer F.Cu) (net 5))
 (segment (start 155.364 87.46) (end 158.476 87.46) (width 0.5) (layer F.Cu) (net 5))
 (segment (start 153.924 88.9) (end 155.364 87.46) (width 0.5) (layer F.Cu) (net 5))
 (segment (start 154.94 118.11) (end 154.94 113.284) (width 0.5) (layer F.Cu) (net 6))
 (segment (start 154.94 113.284) (end 152.908 111.252) (width 0.5) (layer F.Cu) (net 6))
 (segment (start 152.908 111.252) (end 152.908 87.884) (width 0.5) (layer F.Cu) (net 6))
 (segment (start 155.332 85.46) (end 158.476 85.46) (width 0.5) (layer F.Cu) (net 6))
 (segment (start 152.908 87.884) (end 155.332 85.46) (width 0.5) (layer F.Cu) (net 6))
 (segment (start 145.435 91.46) (end 143.276 91.46) (width 0.5) (layer F.Cu) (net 12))
 (segment (start 146.812 92.837) (end 145.435 91.46) (width 0.5) (layer F.Cu) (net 12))
 (segment (start 146.812 107.696) (end 146.812 92.837) (width 0.5) (layer F.Cu) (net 12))
 (segment (start 139.7 118.11) (end 139.7 114.808) (width 0.5) (layer F.Cu) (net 12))
 (segment (start 139.7 114.808) (end 146.812 107.696) (width 0.5) (layer F.Cu) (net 12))
 (segment (start 137.16 115.824) (end 137.16 118.11) (width 0.5) (layer F.Cu) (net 13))
 (segment (start 145.796 107.188) (end 137.16 115.824) (width 0.5) (layer F.Cu) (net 13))
 (segment (start 145.796 94.234) (end 145.796 107.188) (width 0.5) (layer F.Cu) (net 13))
 (segment (start 143.276 93.46) (end 145.022 93.46) (width 0.5) (layer F.Cu) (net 13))
 (segment (start 145.022 93.46) (end 145.796 94.234) (width 0.5) (layer F.Cu) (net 13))
 (segment (start 142.24 118.11) (end 142.24 113.792) (width 0.5) (layer F.Cu) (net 11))
 (segment (start 142.24 113.792) (end 147.828 108.204) (width 0.5) (layer F.Cu) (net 11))
 (segment (start 147.828 108.204) (end 147.828 90.932) (width 0.5) (layer F.Cu) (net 11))
 (segment (start 146.356 89.46) (end 143.276 89.46) (width 0.5) (layer F.Cu) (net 11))
 (segment (start 147.828 90.932) (end 146.356 89.46) (width 0.5) (layer F.Cu) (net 11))
 (segment (start 158.488 93.472) (end 158.476 93.46) (width 0.5) (layer F.Cu) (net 3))
 (segment (start 164.592 93.472) (end 158.488 93.472) (width 0.5) (layer F.Cu) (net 3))
 (segment (start 155.956 108.204) (end 162.56 114.808) (width 0.5) (layer F.Cu) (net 3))
 (segment (start 155.956 94.488) (end 155.956 108.204) (width 0.5) (layer F.Cu) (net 3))
 (segment (start 158.476 93.46) (end 156.984 93.46) (width 0.5) (layer F.Cu) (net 3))
 (segment (start 162.56 114.808) (end 162.56 118.11) (width 0.5) (layer F.Cu) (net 3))
 (segment (start 156.984 93.46) (end 155.956 94.488) (width 0.5) (layer F.Cu) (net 3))
 (segment (start 164.592 93.472) (end 165.354 93.472) (width 0.5) (layer F.Cu) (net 3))
 (segment (start 144.78 118.11) (end 144.78 112.776) (width 0.5) (layer F.Cu) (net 10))
 (segment (start 144.78 112.776) (end 148.844 108.712) (width 0.5) (layer F.Cu) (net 10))
 (segment (start 148.844 108.712) (end 148.844 89.408) (width 0.5) (layer F.Cu) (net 10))
 (segment (start 146.896 87.46) (end 143.276 87.46) (width 0.5) (layer F.Cu) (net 10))
 (segment (start 148.844 89.408) (end 146.896 87.46) (width 0.5) (layer F.Cu) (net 10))
 (segment (start 147.32 118.11) (end 147.32 111.76) (width 0.5) (layer F.Cu) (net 9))
 (segment (start 147.32 111.76) (end 149.86 109.22) (width 0.5) (layer F.Cu) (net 9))
 (segment (start 149.86 109.22) (end 149.86 86.868) (width 0.5) (layer F.Cu) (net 9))
 (segment (start 146.452 83.46) (end 143.276 83.46) (width 0.5) (layer F.Cu) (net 9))
 (segment (start 149.86 86.868) (end 146.452 83.46) (width 0.5) (layer F.Cu) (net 9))
 (segment (start 137.298 85.46) (end 137.16 85.598) (width 0.5) (layer F.Cu) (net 16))
 (segment (start 142.26 85.46) (end 137.298 85.46) (width 0.5) (layer F.Cu) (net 16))
 (segment (start 135.71 81.46) (end 142.26 81.46) (width 0.5) (layer F.Cu) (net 15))
 (segment (start 133.35 83.82) (end 135.71 81.46) (width 0.5) (layer F.Cu) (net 15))
 (segment (start 133.35 85.598) (end 133.35 83.82) (width 0.5) (layer F.Cu) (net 15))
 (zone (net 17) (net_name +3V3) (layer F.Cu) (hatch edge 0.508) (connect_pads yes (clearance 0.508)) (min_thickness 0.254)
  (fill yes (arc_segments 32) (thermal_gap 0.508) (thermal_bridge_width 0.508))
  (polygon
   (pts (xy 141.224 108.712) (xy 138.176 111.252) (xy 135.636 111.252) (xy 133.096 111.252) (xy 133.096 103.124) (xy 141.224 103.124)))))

